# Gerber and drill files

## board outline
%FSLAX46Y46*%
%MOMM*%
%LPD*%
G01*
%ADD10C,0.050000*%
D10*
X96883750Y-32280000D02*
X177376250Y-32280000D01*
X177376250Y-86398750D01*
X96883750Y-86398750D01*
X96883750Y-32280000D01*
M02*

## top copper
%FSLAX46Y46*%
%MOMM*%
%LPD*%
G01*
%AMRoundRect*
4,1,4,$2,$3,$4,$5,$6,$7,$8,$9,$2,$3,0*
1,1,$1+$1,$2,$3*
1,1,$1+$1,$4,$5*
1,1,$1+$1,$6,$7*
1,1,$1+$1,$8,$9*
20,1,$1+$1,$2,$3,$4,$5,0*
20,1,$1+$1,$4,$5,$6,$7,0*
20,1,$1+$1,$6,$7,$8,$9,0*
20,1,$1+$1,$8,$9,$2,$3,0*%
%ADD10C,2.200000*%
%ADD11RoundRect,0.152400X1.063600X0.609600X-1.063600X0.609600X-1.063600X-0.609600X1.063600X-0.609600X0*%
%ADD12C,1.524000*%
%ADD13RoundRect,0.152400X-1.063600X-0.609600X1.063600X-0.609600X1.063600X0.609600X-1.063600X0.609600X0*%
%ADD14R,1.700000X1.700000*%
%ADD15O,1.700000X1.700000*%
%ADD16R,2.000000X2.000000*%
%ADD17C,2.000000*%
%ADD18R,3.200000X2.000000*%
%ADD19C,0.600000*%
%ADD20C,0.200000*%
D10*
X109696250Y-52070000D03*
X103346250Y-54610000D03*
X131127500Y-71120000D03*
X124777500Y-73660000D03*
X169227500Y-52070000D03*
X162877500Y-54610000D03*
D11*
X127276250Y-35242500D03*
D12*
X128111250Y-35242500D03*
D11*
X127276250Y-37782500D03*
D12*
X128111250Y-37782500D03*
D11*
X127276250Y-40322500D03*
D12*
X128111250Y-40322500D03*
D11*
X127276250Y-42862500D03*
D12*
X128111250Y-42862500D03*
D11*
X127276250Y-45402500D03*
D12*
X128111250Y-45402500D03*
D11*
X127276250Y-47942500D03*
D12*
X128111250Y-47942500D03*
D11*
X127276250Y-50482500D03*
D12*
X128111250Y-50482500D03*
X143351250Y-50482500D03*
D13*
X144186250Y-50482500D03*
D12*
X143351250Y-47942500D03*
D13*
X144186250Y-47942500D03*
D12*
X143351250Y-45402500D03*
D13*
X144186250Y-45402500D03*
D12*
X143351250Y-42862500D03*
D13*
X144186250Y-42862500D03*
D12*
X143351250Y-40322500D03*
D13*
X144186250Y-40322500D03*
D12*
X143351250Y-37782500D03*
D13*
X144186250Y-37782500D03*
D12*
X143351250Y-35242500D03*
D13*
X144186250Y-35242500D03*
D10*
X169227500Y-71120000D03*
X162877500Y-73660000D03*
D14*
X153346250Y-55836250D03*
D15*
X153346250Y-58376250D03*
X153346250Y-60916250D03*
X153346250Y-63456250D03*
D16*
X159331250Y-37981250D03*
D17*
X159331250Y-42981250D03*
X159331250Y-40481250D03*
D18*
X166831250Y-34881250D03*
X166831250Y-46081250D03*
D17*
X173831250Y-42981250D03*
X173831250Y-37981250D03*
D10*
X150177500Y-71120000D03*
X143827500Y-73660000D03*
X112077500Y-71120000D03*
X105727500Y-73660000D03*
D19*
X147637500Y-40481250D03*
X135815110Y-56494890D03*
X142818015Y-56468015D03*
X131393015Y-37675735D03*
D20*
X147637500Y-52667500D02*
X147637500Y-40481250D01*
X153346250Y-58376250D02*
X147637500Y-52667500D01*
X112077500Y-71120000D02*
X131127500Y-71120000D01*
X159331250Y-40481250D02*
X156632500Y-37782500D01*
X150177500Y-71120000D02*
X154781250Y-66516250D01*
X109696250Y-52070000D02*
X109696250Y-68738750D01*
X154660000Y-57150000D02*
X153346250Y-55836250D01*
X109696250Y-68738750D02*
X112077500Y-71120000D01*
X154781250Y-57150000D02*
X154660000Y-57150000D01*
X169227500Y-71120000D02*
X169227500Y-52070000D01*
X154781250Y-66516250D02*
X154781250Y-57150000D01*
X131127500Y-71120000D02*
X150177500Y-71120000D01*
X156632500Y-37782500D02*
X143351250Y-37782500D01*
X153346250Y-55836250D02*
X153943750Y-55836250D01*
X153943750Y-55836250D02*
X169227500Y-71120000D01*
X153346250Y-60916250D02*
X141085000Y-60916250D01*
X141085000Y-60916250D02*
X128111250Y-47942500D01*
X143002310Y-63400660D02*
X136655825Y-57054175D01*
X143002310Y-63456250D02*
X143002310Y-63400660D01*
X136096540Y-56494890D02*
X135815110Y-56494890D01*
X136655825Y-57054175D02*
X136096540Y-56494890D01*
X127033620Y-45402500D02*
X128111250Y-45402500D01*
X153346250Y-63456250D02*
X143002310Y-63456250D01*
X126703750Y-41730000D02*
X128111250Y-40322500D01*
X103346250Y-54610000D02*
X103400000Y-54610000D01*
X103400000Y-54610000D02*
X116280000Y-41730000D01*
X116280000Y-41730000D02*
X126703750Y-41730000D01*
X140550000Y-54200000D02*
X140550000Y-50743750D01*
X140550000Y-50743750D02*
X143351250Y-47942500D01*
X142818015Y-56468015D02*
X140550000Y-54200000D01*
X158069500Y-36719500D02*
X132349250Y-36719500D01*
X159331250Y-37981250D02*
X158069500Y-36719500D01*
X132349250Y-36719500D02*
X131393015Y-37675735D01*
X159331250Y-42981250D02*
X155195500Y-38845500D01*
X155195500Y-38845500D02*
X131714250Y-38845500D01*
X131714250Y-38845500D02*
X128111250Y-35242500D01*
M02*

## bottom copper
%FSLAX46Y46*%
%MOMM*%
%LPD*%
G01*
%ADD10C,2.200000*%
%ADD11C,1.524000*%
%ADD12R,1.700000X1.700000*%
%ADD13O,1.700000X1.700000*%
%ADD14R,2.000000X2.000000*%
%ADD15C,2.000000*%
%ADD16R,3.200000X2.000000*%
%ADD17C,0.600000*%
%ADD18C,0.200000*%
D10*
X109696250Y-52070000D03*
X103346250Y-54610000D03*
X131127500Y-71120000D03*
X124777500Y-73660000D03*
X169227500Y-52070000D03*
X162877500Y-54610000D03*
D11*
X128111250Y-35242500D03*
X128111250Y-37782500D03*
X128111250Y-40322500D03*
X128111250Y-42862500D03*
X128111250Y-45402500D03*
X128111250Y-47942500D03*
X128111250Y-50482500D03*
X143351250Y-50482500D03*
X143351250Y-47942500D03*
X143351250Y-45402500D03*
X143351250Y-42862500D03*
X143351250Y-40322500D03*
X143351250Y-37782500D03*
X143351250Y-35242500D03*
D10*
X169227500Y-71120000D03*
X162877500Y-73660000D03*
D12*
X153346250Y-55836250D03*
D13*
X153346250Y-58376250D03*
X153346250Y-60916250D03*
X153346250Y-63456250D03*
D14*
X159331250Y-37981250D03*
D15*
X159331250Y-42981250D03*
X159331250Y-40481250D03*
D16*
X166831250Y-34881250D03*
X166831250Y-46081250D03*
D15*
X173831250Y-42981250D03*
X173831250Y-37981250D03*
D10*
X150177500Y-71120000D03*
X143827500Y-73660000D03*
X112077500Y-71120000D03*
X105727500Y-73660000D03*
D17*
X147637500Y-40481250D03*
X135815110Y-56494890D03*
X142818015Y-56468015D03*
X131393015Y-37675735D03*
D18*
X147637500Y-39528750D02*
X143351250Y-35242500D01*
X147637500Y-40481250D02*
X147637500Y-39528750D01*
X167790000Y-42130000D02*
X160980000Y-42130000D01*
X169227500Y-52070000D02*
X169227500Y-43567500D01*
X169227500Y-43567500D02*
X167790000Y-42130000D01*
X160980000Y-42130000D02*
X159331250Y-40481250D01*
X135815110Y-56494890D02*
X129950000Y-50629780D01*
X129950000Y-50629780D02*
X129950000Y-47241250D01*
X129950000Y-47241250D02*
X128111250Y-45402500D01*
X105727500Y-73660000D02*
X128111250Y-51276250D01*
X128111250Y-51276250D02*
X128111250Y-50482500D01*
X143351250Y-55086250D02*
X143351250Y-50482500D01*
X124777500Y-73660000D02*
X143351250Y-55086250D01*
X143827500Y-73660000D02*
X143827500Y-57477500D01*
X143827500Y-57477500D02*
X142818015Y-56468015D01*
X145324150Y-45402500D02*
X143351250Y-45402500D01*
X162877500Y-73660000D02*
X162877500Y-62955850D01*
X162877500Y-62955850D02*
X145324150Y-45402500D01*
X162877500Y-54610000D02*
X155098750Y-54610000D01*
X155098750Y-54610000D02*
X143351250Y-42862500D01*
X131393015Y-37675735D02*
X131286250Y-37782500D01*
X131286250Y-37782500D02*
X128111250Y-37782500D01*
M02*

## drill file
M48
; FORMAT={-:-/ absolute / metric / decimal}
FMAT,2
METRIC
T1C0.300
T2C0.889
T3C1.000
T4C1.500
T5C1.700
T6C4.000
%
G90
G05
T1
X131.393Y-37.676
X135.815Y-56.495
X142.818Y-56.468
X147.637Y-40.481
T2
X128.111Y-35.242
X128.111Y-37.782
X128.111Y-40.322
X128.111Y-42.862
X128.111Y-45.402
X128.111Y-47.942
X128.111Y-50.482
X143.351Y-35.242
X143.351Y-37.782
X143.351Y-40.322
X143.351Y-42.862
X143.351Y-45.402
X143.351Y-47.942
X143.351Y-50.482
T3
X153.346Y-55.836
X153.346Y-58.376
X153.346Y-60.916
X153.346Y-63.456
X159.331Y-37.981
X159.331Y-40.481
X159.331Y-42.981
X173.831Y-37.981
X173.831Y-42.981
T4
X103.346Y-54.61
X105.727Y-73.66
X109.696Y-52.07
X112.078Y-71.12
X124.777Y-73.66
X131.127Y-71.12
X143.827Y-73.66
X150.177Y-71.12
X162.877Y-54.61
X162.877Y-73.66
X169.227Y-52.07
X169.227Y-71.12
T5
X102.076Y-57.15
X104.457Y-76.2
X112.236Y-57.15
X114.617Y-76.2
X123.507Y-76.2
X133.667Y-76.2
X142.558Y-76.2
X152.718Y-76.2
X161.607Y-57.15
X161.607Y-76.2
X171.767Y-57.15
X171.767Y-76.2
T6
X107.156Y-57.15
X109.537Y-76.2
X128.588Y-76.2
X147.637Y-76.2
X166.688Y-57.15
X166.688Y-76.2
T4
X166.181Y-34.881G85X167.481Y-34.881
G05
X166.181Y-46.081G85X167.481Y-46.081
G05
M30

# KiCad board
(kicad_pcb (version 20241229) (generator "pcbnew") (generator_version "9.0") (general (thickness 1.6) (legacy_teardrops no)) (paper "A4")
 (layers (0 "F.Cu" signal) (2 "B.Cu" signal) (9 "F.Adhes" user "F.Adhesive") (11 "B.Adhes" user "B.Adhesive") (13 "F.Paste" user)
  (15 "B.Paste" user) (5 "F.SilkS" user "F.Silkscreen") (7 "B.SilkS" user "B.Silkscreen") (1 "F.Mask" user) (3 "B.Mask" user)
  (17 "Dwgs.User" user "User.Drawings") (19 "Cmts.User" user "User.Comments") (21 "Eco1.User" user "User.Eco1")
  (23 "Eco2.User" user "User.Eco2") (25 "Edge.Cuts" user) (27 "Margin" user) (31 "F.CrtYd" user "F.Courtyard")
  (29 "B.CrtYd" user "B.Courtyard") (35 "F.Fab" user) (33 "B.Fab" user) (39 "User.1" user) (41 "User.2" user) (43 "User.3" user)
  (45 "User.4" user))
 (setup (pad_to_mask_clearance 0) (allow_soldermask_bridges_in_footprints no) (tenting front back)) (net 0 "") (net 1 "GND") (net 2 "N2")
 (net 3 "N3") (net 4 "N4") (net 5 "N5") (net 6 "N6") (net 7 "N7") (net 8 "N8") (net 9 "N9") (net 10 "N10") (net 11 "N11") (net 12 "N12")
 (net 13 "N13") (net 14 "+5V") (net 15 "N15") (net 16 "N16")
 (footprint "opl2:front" (layer "F.Cu") (at 104.86 38.67)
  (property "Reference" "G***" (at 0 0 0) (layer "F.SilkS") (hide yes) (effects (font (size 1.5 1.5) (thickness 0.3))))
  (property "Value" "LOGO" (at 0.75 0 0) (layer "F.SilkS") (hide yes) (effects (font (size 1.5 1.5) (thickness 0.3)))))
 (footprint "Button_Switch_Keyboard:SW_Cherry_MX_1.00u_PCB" (layer "F.Cu") (at 109.69625 52.07)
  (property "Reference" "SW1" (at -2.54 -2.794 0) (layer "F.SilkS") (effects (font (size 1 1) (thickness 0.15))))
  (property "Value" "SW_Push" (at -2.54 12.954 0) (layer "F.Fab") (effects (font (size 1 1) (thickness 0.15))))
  (pad "" np_thru_hole circle (at -7.62 5.08) (size 1.7 1.7) (drill 1.7) (layers "*.Cu" "*.Mask"))
  (pad "" np_thru_hole circle (at -2.54 5.08) (size 4 4) (drill 4) (layers "*.Cu" "*.Mask"))
  (pad "" np_thru_hole circle (at 2.54 5.08) (size 1.7 1.7) (drill 1.7) (layers "*.Cu" "*.Mask"))
  (pad "1" thru_hole circle (at 0 0) (size 2.2 2.2) (drill 1.5) (layers "*.Cu" "*.Mask") (remove_unused_layers no) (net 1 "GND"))
  (pad "2" thru_hole circle (at -6.35 2.54) (size 2.2 2.2) (drill 1.5) (layers "*.Cu" "*.Mask") (remove_unused_layers no) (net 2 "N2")))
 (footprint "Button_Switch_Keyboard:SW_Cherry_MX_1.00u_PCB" (layer "F.Cu") (at 131.1275 71.12)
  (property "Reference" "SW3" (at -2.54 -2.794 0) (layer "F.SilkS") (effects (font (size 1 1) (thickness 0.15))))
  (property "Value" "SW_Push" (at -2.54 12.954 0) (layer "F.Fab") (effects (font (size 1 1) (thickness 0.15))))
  (pad "" np_thru_hole circle (at -7.62 5.08) (size 1.7 1.7) (drill 1.7) (layers "*.Cu" "*.Mask"))
  (pad "" np_thru_hole circle (at -2.54 5.08) (size 4 4) (drill 4) (layers "*.Cu" "*.Mask"))
  (pad "" np_thru_hole circle (at 2.54 5.08) (size 1.7 1.7) (drill 1.7) (layers "*.Cu" "*.Mask"))
  (pad "1" thru_hole circle (at 0 0) (size 2.2 2.2) (drill 1.5) (layers "*.Cu" "*.Mask") (remove_unused_layers no) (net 1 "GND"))
  (pad "2" thru_hole circle (at -6.35 2.54) (size 2.2 2.2) (drill 1.5) (layers "*.Cu" "*.Mask") (remove_unused_layers no) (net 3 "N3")))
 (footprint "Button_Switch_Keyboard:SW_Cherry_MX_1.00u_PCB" (layer "F.Cu") (at 169.2275 52.07)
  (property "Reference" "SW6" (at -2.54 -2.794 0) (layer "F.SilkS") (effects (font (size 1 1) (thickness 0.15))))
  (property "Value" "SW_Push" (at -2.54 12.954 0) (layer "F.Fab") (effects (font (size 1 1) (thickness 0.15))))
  (pad "" np_thru_hole circle (at -7.62 5.08) (size 1.7 1.7) (drill 1.7) (layers "*.Cu" "*.Mask"))
  (pad "" np_thru_hole circle (at -2.54 5.08) (size 4 4) (drill 4) (layers "*.Cu" "*.Mask"))
  (pad "" np_thru_hole circle (at 2.54 5.08) (size 1.7 1.7) (drill 1.7) (layers "*.Cu" "*.Mask"))
  (pad "1" thru_hole circle (at 0 0) (size 2.2 2.2) (drill 1.5) (layers "*.Cu" "*.Mask") (remove_unused_layers no) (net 1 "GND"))
  (pad "2" thru_hole circle (at -6.35 2.54) (size 2.2 2.2) (drill 1.5) (layers "*.Cu" "*.Mask") (remove_unused_layers no) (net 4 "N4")))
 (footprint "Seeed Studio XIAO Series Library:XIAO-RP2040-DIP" (layer "F.Cu") (at 135.73125 42.8625)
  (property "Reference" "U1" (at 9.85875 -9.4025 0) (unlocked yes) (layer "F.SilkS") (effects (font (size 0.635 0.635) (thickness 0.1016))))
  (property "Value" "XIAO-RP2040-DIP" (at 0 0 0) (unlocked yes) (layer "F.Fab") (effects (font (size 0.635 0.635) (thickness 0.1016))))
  (pad "1" smd roundrect (at -8.455 -7.62 180) (size 2.432 1.524) (layers "F.Cu" "F.Mask") (roundrect_rratio 0.1) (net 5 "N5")
   (thermal_bridge_angle 45))
  (pad "1" thru_hole circle (at -7.62 -7.62 180) (size 1.524 1.524) (drill 0.889) (layers "*.Cu" "*.Mask") (remove_unused_layers no)
   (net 5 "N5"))
  (pad "2" smd roundrect (at -8.455 -5.08 180) (size 2.432 1.524) (layers "F.Cu" "F.Mask") (roundrect_rratio 0.1) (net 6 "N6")
   (thermal_bridge_angle 45))
  (pad "2" thru_hole circle (at -7.62 -5.08 180) (size 1.524 1.524) (drill 0.889) (layers "*.Cu" "*.Mask") (remove_unused_layers no)
   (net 6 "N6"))
  (pad "3" smd roundrect (at -8.455 -2.54 180) (size 2.432 1.524) (layers "F.Cu" "F.Mask") (roundrect_rratio 0.1) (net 2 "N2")
   (thermal_bridge_angle 45))
  (pad "3" thru_hole circle (at -7.62 -2.54 180) (size 1.524 1.524) (drill 0.889) (layers "*.Cu" "*.Mask") (remove_unused_layers no)
   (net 2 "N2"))
  (pad "4" smd roundrect (at -8.455 0 180) (size 2.432 1.524) (layers "F.Cu" "F.Mask") (roundrect_rratio 0.1) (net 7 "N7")
   (thermal_bridge_angle 45))
  (pad "4" thru_hole circle (at -7.62 0 180) (size 1.524 1.524) (drill 0.889) (layers "*.Cu" "*.Mask") (remove_unused_layers no)
   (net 7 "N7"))
  (pad "5" smd roundrect (at -8.455 2.54 180) (size 2.432 1.524) (layers "F.Cu" "F.Mask") (roundrect_rratio 0.1) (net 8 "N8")
   (thermal_bridge_angle 45))
  (pad "5" thru_hole circle (at -7.62 2.54 180) (size 1.524 1.524) (drill 0.889) (layers "*.Cu" "*.Mask") (remove_unused_layers no)
   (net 8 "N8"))
  (pad "6" smd roundrect (at -8.455 5.08 180) (size 2.432 1.524) (layers "F.Cu" "F.Mask") (roundrect_rratio 0.1) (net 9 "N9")
   (thermal_bridge_angle 45))
  (pad "6" thru_hole circle (at -7.62 5.08 180) (size 1.524 1.524) (drill 0.889) (layers "*.Cu" "*.Mask") (remove_unused_layers no)
   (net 9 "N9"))
  (pad "7" smd roundrect (at -8.455 7.62 180) (size 2.432 1.524) (layers "F.Cu" "F.Mask") (roundrect_rratio 0.1) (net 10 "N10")
   (thermal_bridge_angle 45))
  (pad "7" thru_hole circle (at -7.62 7.62 180) (size 1.524 1.524) (drill 0.889) (layers "*.Cu" "*.Mask") (remove_unused_layers no)
   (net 10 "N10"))
  (pad "8" thru_hole circle (at 7.62 7.62) (size 1.524 1.524) (drill 0.889) (layers "*.Cu" "*.Mask") (remove_unused_layers no) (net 3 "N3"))
  (pad "8" smd roundrect (at 8.455 7.62) (size 2.432 1.524) (layers "F.Cu" "F.Mask") (roundrect_rratio 0.1) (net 3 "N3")
   (thermal_bridge_angle 45))
  (pad "9" thru_hole circle (at 7.62 5.08) (size 1.524 1.524) (drill 0.889) (layers "*.Cu" "*.Mask") (remove_unused_layers no)
   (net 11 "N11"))
  (pad "9" smd roundrect (at 8.455 5.08) (size 2.432 1.524) (layers "F.Cu" "F.Mask") (roundrect_rratio 0.1) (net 11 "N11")
   (thermal_bridge_angle 45))
  (pad "10" thru_hole circle (at 7.62 2.54) (size 1.524 1.524) (drill 0.889) (layers "*.Cu" "*.Mask") (remove_unused_layers no)
   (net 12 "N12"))
  (pad "10" smd roundrect (at 8.455 2.54) (size 2.432 1.524) (layers "F.Cu" "F.Mask") (roundrect_rratio 0.1) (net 12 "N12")
   (thermal_bridge_angle 45))
  (pad "11" thru_hole circle (at 7.62 0) (size 1.524 1.524) (drill 0.889) (layers "*.Cu" "*.Mask") (remove_unused_layers no) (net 4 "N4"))
  (pad "11" smd roundrect (at 8.455 0) (size 2.432 1.524) (layers "F.Cu" "F.Mask") (roundrect_rratio 0.1) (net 4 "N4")
   (thermal_bridge_angle 45))
  (pad "12" thru_hole circle (at 7.62 -2.54) (size 1.524 1.524) (drill 0.889) (layers "*.Cu" "*.Mask") (remove_unused_layers no)
   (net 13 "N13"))
  (pad "12" smd roundrect (at 8.455 -2.54) (size 2.432 1.524) (layers "F.Cu" "F.Mask") (roundrect_rratio 0.1) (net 13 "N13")
   (thermal_bridge_angle 45))
  (pad "13" thru_hole circle (at 7.62 -5.08) (size 1.524 1.524) (drill 0.889) (layers "*.Cu" "*.Mask") (remove_unused_layers no)
   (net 1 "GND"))
  (pad "13" smd roundrect (at 8.455 -5.08) (size 2.432 1.524) (layers "F.Cu" "F.Mask") (roundrect_rratio 0.1) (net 1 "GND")
   (thermal_bridge_angle 45))
  (pad "14" thru_hole circle (at 7.62 -7.62) (size 1.524 1.524) (drill 0.889) (layers "*.Cu" "*.Mask") (remove_unused_layers no)
   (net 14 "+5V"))
  (pad "14" smd roundrect (at 8.455 -7.62) (size 2.432 1.524) (layers "F.Cu" "F.Mask") (roundrect_rratio 0.1) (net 14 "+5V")
   (thermal_bridge_angle 45)))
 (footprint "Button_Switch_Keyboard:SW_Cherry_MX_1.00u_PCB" (layer "F.Cu") (at 169.2275 71.12)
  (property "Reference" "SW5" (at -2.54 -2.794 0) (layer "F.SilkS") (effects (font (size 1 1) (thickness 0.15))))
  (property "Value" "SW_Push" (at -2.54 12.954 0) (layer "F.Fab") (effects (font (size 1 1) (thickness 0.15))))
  (pad "" np_thru_hole circle (at -7.62 5.08) (size 1.7 1.7) (drill 1.7) (layers "*.Cu" "*.Mask"))
  (pad "" np_thru_hole circle (at -2.54 5.08) (size 4 4) (drill 4) (layers "*.Cu" "*.Mask"))
  (pad "" np_thru_hole circle (at 2.54 5.08) (size 1.7 1.7) (drill 1.7) (layers "*.Cu" "*.Mask"))
  (pad "1" thru_hole circle (at 0 0) (size 2.2 2.2) (drill 1.5) (layers "*.Cu" "*.Mask") (remove_unused_layers no) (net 1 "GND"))
  (pad "2" thru_hole circle (at -6.35 2.54) (size 2.2 2.2) (drill 1.5) (layers "*.Cu" "*.Mask") (remove_unused_layers no) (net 12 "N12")))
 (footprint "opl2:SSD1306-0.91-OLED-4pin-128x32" (layer "F.Cu") (at 116.84625 53.64625)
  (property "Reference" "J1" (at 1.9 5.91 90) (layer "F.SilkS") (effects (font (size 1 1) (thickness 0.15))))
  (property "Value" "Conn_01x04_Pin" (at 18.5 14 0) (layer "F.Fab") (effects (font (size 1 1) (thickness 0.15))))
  (pad "1" thru_hole rect (at 36.5 2.19) (size 1.7 1.7) (drill 1) (layers "*.Cu" "*.Mask") (remove_unused_layers no) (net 1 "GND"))
  (pad "2" thru_hole oval (at 36.5 4.73) (size 1.7 1.7) (drill 1) (layers "*.Cu" "*.Mask") (remove_unused_layers no) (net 14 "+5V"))
  (pad "3" thru_hole oval (at 36.5 7.27) (size 1.7 1.7) (drill 1) (layers "*.Cu" "*.Mask") (remove_unused_layers no) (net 9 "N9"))
  (pad "4" thru_hole oval (at 36.5 9.81) (size 1.7 1.7) (drill 1) (layers "*.Cu" "*.Mask") (remove_unused_layers no) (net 8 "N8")))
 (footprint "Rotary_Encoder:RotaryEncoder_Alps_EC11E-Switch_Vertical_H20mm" (layer "F.Cu") (at 159.33125 37.98125)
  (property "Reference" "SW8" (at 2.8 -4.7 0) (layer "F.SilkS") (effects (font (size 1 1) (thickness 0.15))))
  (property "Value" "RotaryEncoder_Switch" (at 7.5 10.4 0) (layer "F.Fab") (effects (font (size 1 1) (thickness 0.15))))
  (pad "A" thru_hole rect (at 0 0) (size 2 2) (drill 1) (layers "*.Cu" "*.Mask") (remove_unused_layers no) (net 6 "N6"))
  (pad "B" thru_hole circle (at 0 5) (size 2 2) (drill 1) (layers "*.Cu" "*.Mask") (remove_unused_layers no) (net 5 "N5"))
  (pad "C" thru_hole circle (at 0 2.5) (size 2 2) (drill 1) (layers "*.Cu" "*.Mask") (remove_unused_layers no) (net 1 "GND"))
  (pad "MP" thru_hole rect (at 7.5 -3.1) (size 3.2 2) (drill oval 2.8 1.5) (layers "*.Cu" "*.Mask") (remove_unused_layers no))
  (pad "MP" thru_hole rect (at 7.5 8.1) (size 3.2 2) (drill oval 2.8 1.5) (layers "*.Cu" "*.Mask") (remove_unused_layers no))
  (pad "S1" thru_hole circle (at 14.5 5) (size 2 2) (drill 1) (layers "*.Cu" "*.Mask") (remove_unused_layers no) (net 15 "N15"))
  (pad "S2" thru_hole circle (at 14.5 0) (size 2 2) (drill 1) (layers "*.Cu" "*.Mask") (remove_unused_layers no) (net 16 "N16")))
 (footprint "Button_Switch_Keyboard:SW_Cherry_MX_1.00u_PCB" (layer "F.Cu") (at 150.1775 71.12)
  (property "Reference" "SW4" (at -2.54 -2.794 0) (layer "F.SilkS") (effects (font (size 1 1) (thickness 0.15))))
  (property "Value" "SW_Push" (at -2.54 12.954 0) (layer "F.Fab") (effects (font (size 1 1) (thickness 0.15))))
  (pad "" np_thru_hole circle (at -7.62 5.08) (size 1.7 1.7) (drill 1.7) (layers "*.Cu" "*.Mask"))
  (pad "" np_thru_hole circle (at -2.54 5.08) (size 4 4) (drill 4) (layers "*.Cu" "*.Mask"))
  (pad "" np_thru_hole circle (at 2.54 5.08) (size 1.7 1.7) (drill 1.7) (layers "*.Cu" "*.Mask"))
  (pad "1" thru_hole circle (at 0 0) (size 2.2 2.2) (drill 1.5) (layers "*.Cu" "*.Mask") (remove_unused_layers no) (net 1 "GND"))
  (pad "2" thru_hole circle (at -6.35 2.54) (size 2.2 2.2) (drill 1.5) (layers "*.Cu" "*.Mask") (remove_unused_layers no) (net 11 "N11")))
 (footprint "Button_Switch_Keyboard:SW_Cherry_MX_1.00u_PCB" (layer "F.Cu") (at 112.0775 71.12)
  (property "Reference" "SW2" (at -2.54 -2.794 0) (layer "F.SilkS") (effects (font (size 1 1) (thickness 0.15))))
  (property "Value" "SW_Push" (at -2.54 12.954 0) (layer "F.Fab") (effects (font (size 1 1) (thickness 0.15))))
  (pad "" np_thru_hole circle (at -7.62 5.08) (size 1.7 1.7) (drill 1.7) (layers "*.Cu" "*.Mask"))
  (pad "" np_thru_hole circle (at -2.54 5.08) (size 4 4) (drill 4) (layers "*.Cu" "*.Mask"))
  (pad "" np_thru_hole circle (at 2.54 5.08) (size 1.7 1.7) (drill 1.7) (layers "*.Cu" "*.Mask"))
  (pad "1" thru_hole circle (at 0 0) (size 2.2 2.2) (drill 1.5) (layers "*.Cu" "*.Mask") (remove_unused_layers no) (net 1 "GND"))
  (pad "2" thru_hole circle (at -6.35 2.54) (size 2.2 2.2) (drill 1.5) (layers "*.Cu" "*.Mask") (remove_unused_layers no) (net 10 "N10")))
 (gr_rect (start 96.88375 32.28) (end 177.37625 86.39875) (stroke (width 0.05) (type default)) (fill no) (layer "Edge.Cuts"))
 (segment (start 147.6375 52.6675) (end 147.6375 40.48125) (width 0.2) (layer "F.Cu") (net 14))
 (segment (start 153.34625 58.37625) (end 147.6375 52.6675) (width 0.2) (layer "F.Cu") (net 14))
 (via (at 147.6375 40.48125) (size 0.6) (drill 0.3) (layers "F.Cu" "B.Cu") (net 14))
 (segment (start 147.6375 39.52875) (end 143.35125 35.2425) (width 0.2) (layer "B.Cu") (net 14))
 (segment (start 147.6375 40.48125) (end 147.6375 39.52875) (width 0.2) (layer "B.Cu") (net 14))
 (segment (start 112.0775 71.12) (end 131.1275 71.12) (width 0.2) (layer "F.Cu") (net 1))
 (segment (start 159.33125 40.48125) (end 156.6325 37.7825) (width 0.2) (layer "F.Cu") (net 1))
 (segment (start 150.1775 71.12) (end 154.78125 66.51625) (width 0.2) (layer "F.Cu") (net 1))
 (segment (start 109.69625 52.07) (end 109.69625 68.73875) (width 0.2) (layer "F.Cu") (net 1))
 (segment (start 154.66 57.15) (end 153.34625 55.83625) (width 0.2) (layer "F.Cu") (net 1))
 (segment (start 109.69625 68.73875) (end 112.0775 71.12) (width 0.2) (layer "F.Cu") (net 1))
 (segment (start 154.78125 57.15) (end 154.66 57.15) (width 0.2) (layer "F.Cu") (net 1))
 (segment (start 169.2275 71.12) (end 169.2275 52.07) (width 0.2) (layer "F.Cu") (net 1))
 (segment (start 154.78125 66.51625) (end 154.78125 57.15) (width 0.2) (layer "F.Cu") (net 1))
 (segment (start 131.1275 71.12) (end 150.1775 71.12) (width 0.2) (layer "F.Cu") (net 1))
 (segment (start 156.6325 37.7825) (end 143.35125 37.7825) (width 0.2) (layer "F.Cu") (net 1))
 (segment (start 153.34625 55.83625) (end 153.94375 55.83625) (width 0.2) (layer "F.Cu") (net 1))
 (segment (start 153.94375 55.83625) (end 169.2275 71.12) (width 0.2) (layer "F.Cu") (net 1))
 (segment (start 167.79 42.13) (end 160.98 42.13) (width 0.2) (layer "B.Cu") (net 1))
 (segment (start 169.2275 52.07) (end 169.2275 43.5675) (width 0.2) (layer "B.Cu") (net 1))
 (segment (start 169.2275 43.5675) (end 167.79 42.13) (width 0.2) (layer "B.Cu") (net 1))
 (segment (start 160.98 42.13) (end 159.33125 40.48125) (width 0.2) (layer "B.Cu") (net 1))
 (segment (start 153.34625 60.91625) (end 141.085 60.91625) (width 0.2) (layer "F.Cu") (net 9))
 (segment (start 141.085 60.91625) (end 128.11125 47.9425) (width 0.2) (layer "F.Cu") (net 9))
 (segment (start 143.00231 63.40066) (end 136.655825 57.054175) (width 0.2) (layer "F.Cu") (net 8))
 (segment (start 143.00231 63.45625) (end 143.00231 63.40066) (width 0.2) (layer "F.Cu") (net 8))
 (segment (start 136.09654 56.49489) (end 135.81511 56.49489) (width 0.2) (layer "F.Cu") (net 8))
 (segment (start 136.655825 57.054175) (end 136.09654 56.49489) (width 0.2) (layer "F.Cu") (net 8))
 (segment (start 127.03362 45.4025) (end 128.11125 45.4025) (width 0.2) (layer "F.Cu") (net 8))
 (segment (start 153.34625 63.45625) (end 143.00231 63.45625) (width 0.2) (layer "F.Cu") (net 8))
 (via (at 135.81511 56.49489) (size 0.6) (drill 0.3) (layers "F.Cu" "B.Cu") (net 8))
 (segment (start 135.81511 56.49489) (end 129.95 50.62978) (width 0.2) (layer "B.Cu") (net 8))
 (segment (start 129.95 50.62978) (end 129.95 47.24125) (width 0.2) (layer "B.Cu") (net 8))
 (segment (start 129.95 47.24125) (end 128.11125 45.4025) (width 0.2) (layer "B.Cu") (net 8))
 (segment (start 126.70375 41.73) (end 128.11125 40.3225) (width 0.2) (layer "F.Cu") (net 2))
 (segment (start 103.34625 54.61) (end 103.4 54.61) (width 0.2) (layer "F.Cu") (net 2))
 (segment (start 103.4 54.61) (end 116.28 41.73) (width 0.2) (layer "F.Cu") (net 2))
 (segment (start 116.28 41.73) (end 126.70375 41.73) (width 0.2) (layer "F.Cu") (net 2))
 (segment (start 105.7275 73.66) (end 128.11125 51.27625) (width 0.2) (layer "B.Cu") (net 10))
 (segment (start 128.11125 51.27625) (end 128.11125 50.4825) (width 0.2) (layer "B.Cu") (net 10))
 (segment (start 143.35125 55.08625) (end 143.35125 50.4825) (width 0.2) (layer "B.Cu") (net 3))
 (segment (start 124.7775 73.66) (end 143.35125 55.08625) (width 0.2) (layer "B.Cu") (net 3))
 (segment (start 140.55 54.2) (end 140.55 50.74375) (width 0.2) (layer "F.Cu") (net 11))
 (segment (start 140.55 50.74375) (end 143.35125 47.9425) (width 0.2) (layer "F.Cu") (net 11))
 (segment (start 142.818015 56.468015) (end 140.55 54.2) (width 0.2) (layer "F.Cu") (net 11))
 (via (at 142.818015 56.468015) (size 0.6) (drill 0.3) (layers "F.Cu" "B.Cu") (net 11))
 (segment (start 143.8275 73.66) (end 143.8275 57.4775) (width 0.2) (layer "B.Cu") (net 11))
 (segment (start 143.8275 57.4775) (end 142.818015 56.468015) (width 0.2) (layer "B.Cu") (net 11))
 (segment (start 145.32415 45.4025) (end 143.35125 45.4025) (width 0.2) (layer "B.Cu") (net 12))
 (segment (start 162.8775 73.66) (end 162.8775 62.95585) (width 0.2) (layer "B.Cu") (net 12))
 (segment (start 162.8775 62.95585) (end 145.32415 45.4025) (width 0.2) (layer "B.Cu") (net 12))
 (segment (start 162.8775 54.61) (end 155.09875 54.61) (width 0.2) (layer "B.Cu") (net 4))
 (segment (start 155.09875 54.61) (end 143.35125 42.8625) (width 0.2) (layer "B.Cu") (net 4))
 (segment (start 158.0695 36.7195) (end 132.34925 36.7195) (width 0.2) (layer "F.Cu") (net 6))
 (segment (start 159.33125 37.98125) (end 158.0695 36.7195) (width 0.2) (layer "F.Cu") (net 6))
 (segment (start 132.34925 36.7195) (end 131.393015 37.675735) (width 0.2) (layer "F.Cu") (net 6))
 (via (at 131.393015 37.675735) (size 0.6) (drill 0.3) (layers "F.Cu" "B.Cu") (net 6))
 (segment (start 131.393015 37.675735) (end 131.28625 37.7825) (width 0.2) (layer "B.Cu") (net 6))
 (segment (start 131.28625 37.7825) (end 128.11125 37.7825) (width 0.2) (layer "B.Cu") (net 6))
 (segment (start 159.33125 42.98125) (end 155.1955 38.8455) (width 0.2) (layer "F.Cu") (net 5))
 (segment (start 155.1955 38.8455) (end 131.71425 38.8455) (width 0.2) (layer "F.Cu") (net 5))
 (segment (start 131.71425 38.8455) (end 128.11125 35.2425) (width 0.2) (layer "F.Cu") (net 5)))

